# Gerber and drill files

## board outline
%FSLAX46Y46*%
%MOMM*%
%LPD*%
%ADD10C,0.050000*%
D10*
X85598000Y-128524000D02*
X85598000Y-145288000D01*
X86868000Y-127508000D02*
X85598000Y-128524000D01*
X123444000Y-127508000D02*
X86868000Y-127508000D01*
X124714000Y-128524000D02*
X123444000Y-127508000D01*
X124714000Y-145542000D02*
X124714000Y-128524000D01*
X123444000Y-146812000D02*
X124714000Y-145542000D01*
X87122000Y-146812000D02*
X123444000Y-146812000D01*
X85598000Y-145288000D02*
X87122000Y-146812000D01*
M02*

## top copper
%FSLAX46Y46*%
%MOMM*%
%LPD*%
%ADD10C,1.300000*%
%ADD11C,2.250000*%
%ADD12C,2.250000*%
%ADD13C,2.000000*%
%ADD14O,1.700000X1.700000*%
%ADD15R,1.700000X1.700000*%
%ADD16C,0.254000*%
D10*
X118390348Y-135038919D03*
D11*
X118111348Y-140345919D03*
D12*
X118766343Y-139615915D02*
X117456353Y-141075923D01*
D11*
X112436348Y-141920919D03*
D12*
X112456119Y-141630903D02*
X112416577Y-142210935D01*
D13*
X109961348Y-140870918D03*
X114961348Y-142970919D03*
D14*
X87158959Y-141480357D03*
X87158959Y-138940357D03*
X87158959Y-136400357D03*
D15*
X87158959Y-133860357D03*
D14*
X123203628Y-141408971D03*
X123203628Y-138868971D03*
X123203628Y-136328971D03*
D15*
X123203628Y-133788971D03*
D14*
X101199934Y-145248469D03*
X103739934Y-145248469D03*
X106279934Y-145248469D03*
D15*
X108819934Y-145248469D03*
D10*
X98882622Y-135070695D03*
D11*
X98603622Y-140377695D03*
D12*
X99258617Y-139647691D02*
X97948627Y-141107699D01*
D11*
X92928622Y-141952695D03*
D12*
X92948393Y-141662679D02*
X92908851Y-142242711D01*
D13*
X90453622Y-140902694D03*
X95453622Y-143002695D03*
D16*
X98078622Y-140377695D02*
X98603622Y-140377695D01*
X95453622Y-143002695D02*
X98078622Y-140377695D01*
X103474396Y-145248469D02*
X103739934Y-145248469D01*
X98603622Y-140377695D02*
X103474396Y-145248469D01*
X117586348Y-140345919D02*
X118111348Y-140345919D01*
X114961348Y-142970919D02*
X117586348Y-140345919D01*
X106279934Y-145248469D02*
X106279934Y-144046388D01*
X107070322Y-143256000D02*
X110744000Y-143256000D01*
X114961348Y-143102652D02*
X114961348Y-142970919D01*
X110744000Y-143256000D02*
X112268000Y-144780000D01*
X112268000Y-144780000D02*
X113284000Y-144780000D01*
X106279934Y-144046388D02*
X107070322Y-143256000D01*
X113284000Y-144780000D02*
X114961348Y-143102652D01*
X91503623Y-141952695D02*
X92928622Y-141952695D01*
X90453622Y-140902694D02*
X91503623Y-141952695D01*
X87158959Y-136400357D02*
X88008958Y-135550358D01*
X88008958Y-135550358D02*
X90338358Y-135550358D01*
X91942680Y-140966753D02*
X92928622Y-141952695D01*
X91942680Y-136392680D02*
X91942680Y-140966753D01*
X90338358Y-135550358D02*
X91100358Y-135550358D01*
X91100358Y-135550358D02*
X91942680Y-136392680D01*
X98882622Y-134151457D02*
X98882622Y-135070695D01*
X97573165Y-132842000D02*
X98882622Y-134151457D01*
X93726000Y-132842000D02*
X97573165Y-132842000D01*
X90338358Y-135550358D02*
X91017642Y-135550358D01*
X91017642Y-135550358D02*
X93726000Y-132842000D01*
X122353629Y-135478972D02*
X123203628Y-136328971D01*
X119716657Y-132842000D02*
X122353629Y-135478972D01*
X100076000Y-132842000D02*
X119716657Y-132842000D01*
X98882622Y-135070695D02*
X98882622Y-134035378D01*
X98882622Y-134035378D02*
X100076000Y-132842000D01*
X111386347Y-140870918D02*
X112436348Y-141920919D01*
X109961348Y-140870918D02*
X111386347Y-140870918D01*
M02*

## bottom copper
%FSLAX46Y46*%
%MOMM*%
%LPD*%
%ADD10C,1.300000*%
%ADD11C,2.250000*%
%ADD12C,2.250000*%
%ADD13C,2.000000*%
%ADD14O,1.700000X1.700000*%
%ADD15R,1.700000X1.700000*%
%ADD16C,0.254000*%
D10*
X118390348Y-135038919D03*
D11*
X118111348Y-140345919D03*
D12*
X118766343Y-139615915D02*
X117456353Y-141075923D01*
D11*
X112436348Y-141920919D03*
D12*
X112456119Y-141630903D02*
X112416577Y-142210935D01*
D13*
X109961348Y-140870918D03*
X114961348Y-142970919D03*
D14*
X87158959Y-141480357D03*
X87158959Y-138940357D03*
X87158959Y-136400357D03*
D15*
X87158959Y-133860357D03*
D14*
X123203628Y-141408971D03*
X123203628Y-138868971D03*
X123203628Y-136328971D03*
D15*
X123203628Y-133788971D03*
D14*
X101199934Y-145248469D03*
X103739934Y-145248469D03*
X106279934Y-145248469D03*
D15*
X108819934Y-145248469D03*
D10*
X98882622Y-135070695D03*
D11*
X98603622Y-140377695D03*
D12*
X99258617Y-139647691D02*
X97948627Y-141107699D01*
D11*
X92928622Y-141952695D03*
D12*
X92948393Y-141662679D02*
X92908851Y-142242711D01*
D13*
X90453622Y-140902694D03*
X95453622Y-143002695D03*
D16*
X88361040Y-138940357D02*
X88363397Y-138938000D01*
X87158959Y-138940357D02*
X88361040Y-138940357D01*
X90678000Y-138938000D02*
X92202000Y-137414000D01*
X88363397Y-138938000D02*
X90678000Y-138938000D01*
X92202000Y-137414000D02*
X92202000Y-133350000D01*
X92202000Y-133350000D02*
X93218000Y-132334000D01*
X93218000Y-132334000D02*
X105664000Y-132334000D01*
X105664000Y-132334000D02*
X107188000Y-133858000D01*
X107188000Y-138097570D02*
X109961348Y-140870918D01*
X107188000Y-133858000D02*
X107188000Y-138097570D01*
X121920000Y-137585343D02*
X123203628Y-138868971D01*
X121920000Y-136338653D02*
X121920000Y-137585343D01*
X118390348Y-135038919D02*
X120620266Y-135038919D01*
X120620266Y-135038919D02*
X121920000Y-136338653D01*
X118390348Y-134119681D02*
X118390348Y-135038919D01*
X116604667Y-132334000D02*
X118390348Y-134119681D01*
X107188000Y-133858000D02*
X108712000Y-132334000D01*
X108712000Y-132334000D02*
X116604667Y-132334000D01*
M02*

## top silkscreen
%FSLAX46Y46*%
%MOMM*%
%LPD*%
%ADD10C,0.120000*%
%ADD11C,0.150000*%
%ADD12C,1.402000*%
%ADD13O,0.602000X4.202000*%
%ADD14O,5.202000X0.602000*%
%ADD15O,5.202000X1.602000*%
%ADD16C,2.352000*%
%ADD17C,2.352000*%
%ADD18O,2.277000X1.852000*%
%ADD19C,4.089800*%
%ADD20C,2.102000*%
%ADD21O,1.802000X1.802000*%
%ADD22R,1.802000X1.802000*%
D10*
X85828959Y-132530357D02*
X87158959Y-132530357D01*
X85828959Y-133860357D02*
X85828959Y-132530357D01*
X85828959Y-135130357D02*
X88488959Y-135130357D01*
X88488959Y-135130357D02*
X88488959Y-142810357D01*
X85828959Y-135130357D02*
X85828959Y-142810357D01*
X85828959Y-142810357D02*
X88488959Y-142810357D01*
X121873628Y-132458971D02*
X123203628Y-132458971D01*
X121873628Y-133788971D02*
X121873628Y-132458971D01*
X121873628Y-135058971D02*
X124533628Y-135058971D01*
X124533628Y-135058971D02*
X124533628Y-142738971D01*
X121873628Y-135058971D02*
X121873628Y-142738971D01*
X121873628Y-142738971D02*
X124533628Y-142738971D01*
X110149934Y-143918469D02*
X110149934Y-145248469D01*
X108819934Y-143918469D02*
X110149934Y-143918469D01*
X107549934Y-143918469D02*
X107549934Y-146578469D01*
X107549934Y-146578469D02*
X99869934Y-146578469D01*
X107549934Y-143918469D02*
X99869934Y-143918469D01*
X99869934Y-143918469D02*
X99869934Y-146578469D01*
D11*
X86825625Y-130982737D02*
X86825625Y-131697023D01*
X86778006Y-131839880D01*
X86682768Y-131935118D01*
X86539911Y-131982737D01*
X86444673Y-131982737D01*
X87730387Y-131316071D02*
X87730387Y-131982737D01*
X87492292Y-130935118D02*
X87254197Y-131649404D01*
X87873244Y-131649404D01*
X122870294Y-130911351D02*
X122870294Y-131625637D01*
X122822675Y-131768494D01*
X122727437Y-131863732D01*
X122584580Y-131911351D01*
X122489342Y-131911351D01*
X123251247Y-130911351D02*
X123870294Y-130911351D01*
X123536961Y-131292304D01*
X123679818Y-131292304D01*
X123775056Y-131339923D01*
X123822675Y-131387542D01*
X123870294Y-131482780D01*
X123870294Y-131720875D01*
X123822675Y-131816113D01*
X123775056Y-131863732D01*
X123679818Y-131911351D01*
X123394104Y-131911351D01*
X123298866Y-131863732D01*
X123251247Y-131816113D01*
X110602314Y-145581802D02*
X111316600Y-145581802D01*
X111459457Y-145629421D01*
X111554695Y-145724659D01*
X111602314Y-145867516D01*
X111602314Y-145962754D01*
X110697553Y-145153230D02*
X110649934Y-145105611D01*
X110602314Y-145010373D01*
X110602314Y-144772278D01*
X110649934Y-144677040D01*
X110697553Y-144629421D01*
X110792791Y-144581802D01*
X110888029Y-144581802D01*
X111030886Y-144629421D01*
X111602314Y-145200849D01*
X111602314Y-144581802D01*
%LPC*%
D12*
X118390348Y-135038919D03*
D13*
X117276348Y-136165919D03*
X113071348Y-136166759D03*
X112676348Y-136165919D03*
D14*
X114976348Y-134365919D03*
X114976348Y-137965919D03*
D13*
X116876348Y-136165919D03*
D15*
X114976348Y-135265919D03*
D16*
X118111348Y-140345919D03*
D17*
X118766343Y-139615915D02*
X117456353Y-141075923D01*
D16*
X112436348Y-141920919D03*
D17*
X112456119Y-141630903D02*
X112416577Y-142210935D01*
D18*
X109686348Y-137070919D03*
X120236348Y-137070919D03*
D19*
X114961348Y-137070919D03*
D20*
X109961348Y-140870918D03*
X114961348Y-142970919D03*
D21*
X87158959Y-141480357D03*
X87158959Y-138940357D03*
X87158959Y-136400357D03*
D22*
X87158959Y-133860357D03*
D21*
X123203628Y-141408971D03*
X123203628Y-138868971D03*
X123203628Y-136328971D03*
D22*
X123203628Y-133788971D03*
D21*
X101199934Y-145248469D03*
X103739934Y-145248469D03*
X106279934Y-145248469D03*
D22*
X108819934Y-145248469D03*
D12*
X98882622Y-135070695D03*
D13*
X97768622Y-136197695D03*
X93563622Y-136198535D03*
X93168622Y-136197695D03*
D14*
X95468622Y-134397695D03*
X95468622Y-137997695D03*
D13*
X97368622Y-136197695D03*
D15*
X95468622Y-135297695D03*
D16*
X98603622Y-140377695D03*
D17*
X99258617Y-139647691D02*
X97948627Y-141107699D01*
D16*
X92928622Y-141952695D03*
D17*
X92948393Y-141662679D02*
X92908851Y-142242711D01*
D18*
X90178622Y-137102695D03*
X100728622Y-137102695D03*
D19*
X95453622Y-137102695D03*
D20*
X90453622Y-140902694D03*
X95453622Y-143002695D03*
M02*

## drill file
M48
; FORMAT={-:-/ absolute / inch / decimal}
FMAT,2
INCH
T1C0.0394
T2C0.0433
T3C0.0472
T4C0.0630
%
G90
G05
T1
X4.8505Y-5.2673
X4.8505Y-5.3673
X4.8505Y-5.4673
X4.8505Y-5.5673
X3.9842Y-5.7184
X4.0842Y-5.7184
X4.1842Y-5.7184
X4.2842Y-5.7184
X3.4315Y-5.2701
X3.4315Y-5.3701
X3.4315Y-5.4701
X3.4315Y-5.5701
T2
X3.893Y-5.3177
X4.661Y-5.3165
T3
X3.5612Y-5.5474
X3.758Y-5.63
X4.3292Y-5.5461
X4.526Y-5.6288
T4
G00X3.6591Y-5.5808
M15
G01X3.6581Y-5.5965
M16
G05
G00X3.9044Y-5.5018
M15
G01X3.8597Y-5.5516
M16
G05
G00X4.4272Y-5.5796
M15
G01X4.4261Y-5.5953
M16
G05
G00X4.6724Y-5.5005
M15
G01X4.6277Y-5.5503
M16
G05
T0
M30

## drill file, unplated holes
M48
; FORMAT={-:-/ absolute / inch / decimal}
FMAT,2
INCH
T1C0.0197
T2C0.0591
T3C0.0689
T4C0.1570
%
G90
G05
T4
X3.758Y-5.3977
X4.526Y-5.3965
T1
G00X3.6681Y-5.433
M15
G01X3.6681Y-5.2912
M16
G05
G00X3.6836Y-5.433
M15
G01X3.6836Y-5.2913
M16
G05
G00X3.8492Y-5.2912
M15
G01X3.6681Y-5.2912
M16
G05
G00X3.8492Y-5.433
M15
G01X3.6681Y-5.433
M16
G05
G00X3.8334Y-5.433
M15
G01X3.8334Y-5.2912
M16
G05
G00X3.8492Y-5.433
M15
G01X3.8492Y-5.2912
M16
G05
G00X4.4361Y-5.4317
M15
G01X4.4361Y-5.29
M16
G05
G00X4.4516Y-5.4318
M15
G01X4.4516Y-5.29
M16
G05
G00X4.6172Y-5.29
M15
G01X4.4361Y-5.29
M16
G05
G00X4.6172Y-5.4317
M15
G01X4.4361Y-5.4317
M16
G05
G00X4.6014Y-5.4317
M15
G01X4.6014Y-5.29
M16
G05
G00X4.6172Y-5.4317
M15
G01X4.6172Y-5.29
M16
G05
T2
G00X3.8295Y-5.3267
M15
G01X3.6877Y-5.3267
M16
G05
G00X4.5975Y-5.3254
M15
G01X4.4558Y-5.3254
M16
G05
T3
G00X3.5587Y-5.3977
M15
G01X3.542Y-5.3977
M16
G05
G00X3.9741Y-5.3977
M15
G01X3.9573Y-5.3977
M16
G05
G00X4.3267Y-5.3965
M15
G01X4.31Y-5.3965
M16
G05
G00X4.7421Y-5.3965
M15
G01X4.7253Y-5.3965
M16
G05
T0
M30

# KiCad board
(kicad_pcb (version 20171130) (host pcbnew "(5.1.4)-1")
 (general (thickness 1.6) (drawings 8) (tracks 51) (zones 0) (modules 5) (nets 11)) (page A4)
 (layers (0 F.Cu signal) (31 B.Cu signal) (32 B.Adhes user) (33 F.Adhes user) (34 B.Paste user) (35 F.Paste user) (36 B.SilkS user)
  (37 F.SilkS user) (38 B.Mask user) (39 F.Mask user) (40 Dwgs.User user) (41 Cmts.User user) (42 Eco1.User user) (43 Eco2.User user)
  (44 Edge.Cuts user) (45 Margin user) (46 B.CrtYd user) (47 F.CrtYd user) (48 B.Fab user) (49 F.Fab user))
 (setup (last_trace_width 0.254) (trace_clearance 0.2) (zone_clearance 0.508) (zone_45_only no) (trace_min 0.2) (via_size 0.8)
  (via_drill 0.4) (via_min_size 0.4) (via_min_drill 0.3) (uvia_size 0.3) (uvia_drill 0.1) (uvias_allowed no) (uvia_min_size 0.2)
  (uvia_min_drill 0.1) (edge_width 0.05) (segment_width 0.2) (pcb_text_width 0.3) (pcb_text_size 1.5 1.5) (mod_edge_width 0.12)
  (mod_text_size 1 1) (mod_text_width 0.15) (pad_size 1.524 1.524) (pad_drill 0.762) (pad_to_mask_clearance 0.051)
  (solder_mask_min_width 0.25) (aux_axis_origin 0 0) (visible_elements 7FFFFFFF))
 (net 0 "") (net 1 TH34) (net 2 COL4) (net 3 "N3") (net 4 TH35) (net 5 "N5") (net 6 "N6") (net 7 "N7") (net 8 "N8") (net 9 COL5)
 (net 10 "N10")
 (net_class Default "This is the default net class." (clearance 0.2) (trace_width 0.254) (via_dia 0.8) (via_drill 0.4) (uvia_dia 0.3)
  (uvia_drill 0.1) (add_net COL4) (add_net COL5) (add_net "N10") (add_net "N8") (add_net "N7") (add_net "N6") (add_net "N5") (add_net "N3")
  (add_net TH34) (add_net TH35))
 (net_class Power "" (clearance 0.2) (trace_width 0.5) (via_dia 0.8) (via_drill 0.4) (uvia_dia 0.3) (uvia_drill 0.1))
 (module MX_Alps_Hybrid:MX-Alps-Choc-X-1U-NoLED (layer F.Cu) (at 114.961348 137.070919 180)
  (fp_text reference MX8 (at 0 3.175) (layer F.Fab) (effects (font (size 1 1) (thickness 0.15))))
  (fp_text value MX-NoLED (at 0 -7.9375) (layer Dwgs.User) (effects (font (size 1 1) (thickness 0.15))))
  (pad 1 thru_hole circle (at -3.429 2.032 180) (size 1.3 1.3) (drill 1.1) (layers *.Cu *.Mask) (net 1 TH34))
  (pad "" np_thru_hole oval (at -2.315 0.905 180) (size 0.5 4.1) (drill oval 0.5 4.1) (layers *.Cu *.Mask))
  (pad "" np_thru_hole oval (at 1.89 0.90416 180) (size 0.5 4.1) (drill oval 0.5 4.1) (layers *.Cu *.Mask))
  (pad "" np_thru_hole oval (at 2.285 0.905 180) (size 0.5 4.1) (drill oval 0.5 4.1) (layers *.Cu *.Mask))
  (pad "" np_thru_hole oval (at -0.015 2.705 180) (size 5.1 0.5) (drill oval 5.1 0.5) (layers *.Cu *.Mask))
  (pad "" np_thru_hole oval (at -0.015 -0.895 180) (size 5.1 0.5) (drill oval 5.1 0.5) (layers *.Cu *.Mask))
  (pad "" np_thru_hole oval (at -1.915 0.905 180) (size 0.5 4.1) (drill oval 0.5 4.1) (layers *.Cu *.Mask))
  (pad "" np_thru_hole oval (at -0.015 1.805 180) (size 5.1 1.5) (drill oval 5.1 1.5) (layers *.Cu *.Mask))
  (pad 2 thru_hole oval (at -3.15 -3.275 228.1) (size 4.211556 2.25) (drill oval 3.3 1.6) (layers *.Cu *.Mask) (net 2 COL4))
  (pad 1 thru_hole oval (at 2.525 -4.85 266.1) (size 2.831378 2.25) (drill oval 2 1.6) (layers *.Cu *.Mask) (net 1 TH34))
  (pad "" np_thru_hole oval (at 5.275 0 270) (size 1.75 2.175) (drill oval 1.75 2.175) (layers *.Cu *.Mask))
  (pad "" np_thru_hole oval (at -5.275 0 270) (size 1.75 2.175) (drill oval 1.75 2.175) (layers *.Cu *.Mask))
  (pad "" np_thru_hole circle (at 0 0 180) (size 3.9878 3.9878) (drill 3.9878) (layers *.Cu *.Mask))
  (pad 1 thru_hole circle (at 5 -3.799999 180) (size 2 2) (drill 1.2) (layers *.Cu *.Mask) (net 1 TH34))
  (pad 2 thru_hole circle (at 0 -5.9 180) (size 2 2) (drill 1.2) (layers *.Cu *.Mask) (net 2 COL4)))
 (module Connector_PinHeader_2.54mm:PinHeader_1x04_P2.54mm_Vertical (layer F.Cu) (at 87.158959 133.860357)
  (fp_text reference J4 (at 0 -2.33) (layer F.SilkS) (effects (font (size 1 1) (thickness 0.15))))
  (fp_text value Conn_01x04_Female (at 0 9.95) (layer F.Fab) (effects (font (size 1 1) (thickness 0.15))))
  (fp_line (start -1.33 -1.33) (end 0 -1.33) (layer F.SilkS) (width 0.12))
  (fp_line (start -1.33 0) (end -1.33 -1.33) (layer F.SilkS) (width 0.12))
  (fp_line (start -1.33 1.27) (end 1.33 1.27) (layer F.SilkS) (width 0.12))
  (fp_line (start 1.33 1.27) (end 1.33 8.95) (layer F.SilkS) (width 0.12))
  (fp_line (start -1.33 1.27) (end -1.33 8.95) (layer F.SilkS) (width 0.12))
  (fp_line (start -1.33 8.95) (end 1.33 8.95) (layer F.SilkS) (width 0.12))
  (pad 4 thru_hole oval (at 0 7.62) (size 1.7 1.7) (drill 1) (layers *.Cu *.Mask) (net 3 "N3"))
  (pad 3 thru_hole oval (at 0 5.08) (size 1.7 1.7) (drill 1) (layers *.Cu *.Mask) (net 1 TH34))
  (pad 2 thru_hole oval (at 0 2.54) (size 1.7 1.7) (drill 1) (layers *.Cu *.Mask) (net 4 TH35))
  (pad 1 thru_hole rect (at 0 0) (size 1.7 1.7) (drill 1) (layers *.Cu *.Mask) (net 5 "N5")))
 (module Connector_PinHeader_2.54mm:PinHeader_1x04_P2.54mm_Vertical (layer F.Cu) (at 123.203628 133.788971)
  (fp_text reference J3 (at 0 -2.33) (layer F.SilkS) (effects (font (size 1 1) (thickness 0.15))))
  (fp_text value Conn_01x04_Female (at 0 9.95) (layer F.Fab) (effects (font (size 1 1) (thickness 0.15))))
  (fp_line (start -1.33 -1.33) (end 0 -1.33) (layer F.SilkS) (width 0.12))
  (fp_line (start -1.33 0) (end -1.33 -1.33) (layer F.SilkS) (width 0.12))
  (fp_line (start -1.33 1.27) (end 1.33 1.27) (layer F.SilkS) (width 0.12))
  (fp_line (start 1.33 1.27) (end 1.33 8.95) (layer F.SilkS) (width 0.12))
  (fp_line (start -1.33 1.27) (end -1.33 8.95) (layer F.SilkS) (width 0.12))
  (fp_line (start -1.33 8.95) (end 1.33 8.95) (layer F.SilkS) (width 0.12))
  (pad 4 thru_hole oval (at 0 7.62) (size 1.7 1.7) (drill 1) (layers *.Cu *.Mask) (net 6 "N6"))
  (pad 3 thru_hole oval (at 0 5.08) (size 1.7 1.7) (drill 1) (layers *.Cu *.Mask) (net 1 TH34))
  (pad 2 thru_hole oval (at 0 2.54) (size 1.7 1.7) (drill 1) (layers *.Cu *.Mask) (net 4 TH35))
  (pad 1 thru_hole rect (at 0 0) (size 1.7 1.7) (drill 1) (layers *.Cu *.Mask) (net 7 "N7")))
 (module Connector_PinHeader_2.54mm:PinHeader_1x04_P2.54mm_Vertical (layer F.Cu) (at 108.819934 145.248469 270)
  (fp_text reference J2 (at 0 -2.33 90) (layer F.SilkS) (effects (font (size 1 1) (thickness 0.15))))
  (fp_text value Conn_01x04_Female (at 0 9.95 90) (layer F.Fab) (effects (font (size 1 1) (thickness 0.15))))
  (fp_line (start -1.33 -1.33) (end 0 -1.33) (layer F.SilkS) (width 0.12))
  (fp_line (start -1.33 0) (end -1.33 -1.33) (layer F.SilkS) (width 0.12))
  (fp_line (start -1.33 1.27) (end 1.33 1.27) (layer F.SilkS) (width 0.12))
  (fp_line (start 1.33 1.27) (end 1.33 8.95) (layer F.SilkS) (width 0.12))
  (fp_line (start -1.33 1.27) (end -1.33 8.95) (layer F.SilkS) (width 0.12))
  (fp_line (start -1.33 8.95) (end 1.33 8.95) (layer F.SilkS) (width 0.12))
  (pad 4 thru_hole oval (at 0 7.62 270) (size 1.7 1.7) (drill 1) (layers *.Cu *.Mask) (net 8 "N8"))
  (pad 3 thru_hole oval (at 0 5.08 270) (size 1.7 1.7) (drill 1) (layers *.Cu *.Mask) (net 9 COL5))
  (pad 2 thru_hole oval (at 0 2.54 270) (size 1.7 1.7) (drill 1) (layers *.Cu *.Mask) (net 2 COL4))
  (pad 1 thru_hole rect (at 0 0 270) (size 1.7 1.7) (drill 1) (layers *.Cu *.Mask) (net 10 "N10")))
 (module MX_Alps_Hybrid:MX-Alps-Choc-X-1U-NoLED (layer F.Cu) (at 95.453622 137.102695 180)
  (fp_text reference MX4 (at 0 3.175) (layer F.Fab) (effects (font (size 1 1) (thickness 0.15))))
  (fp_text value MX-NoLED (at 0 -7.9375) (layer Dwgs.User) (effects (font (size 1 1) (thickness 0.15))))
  (pad 1 thru_hole circle (at -3.429 2.032 180) (size 1.3 1.3) (drill 1.1) (layers *.Cu *.Mask) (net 4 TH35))
  (pad "" np_thru_hole oval (at -2.315 0.905 180) (size 0.5 4.1) (drill oval 0.5 4.1) (layers *.Cu *.Mask))
  (pad "" np_thru_hole oval (at 1.89 0.90416 180) (size 0.5 4.1) (drill oval 0.5 4.1) (layers *.Cu *.Mask))
  (pad "" np_thru_hole oval (at 2.285 0.905 180) (size 0.5 4.1) (drill oval 0.5 4.1) (layers *.Cu *.Mask))
  (pad "" np_thru_hole oval (at -0.015 2.705 180) (size 5.1 0.5) (drill oval 5.1 0.5) (layers *.Cu *.Mask))
  (pad "" np_thru_hole oval (at -0.015 -0.895 180) (size 5.1 0.5) (drill oval 5.1 0.5) (layers *.Cu *.Mask))
  (pad "" np_thru_hole oval (at -1.915 0.905 180) (size 0.5 4.1) (drill oval 0.5 4.1) (layers *.Cu *.Mask))
  (pad "" np_thru_hole oval (at -0.015 1.805 180) (size 5.1 1.5) (drill oval 5.1 1.5) (layers *.Cu *.Mask))
  (pad 2 thru_hole oval (at -3.15 -3.275 228.1) (size 4.211556 2.25) (drill oval 3.3 1.6) (layers *.Cu *.Mask) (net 9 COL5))
  (pad 1 thru_hole oval (at 2.525 -4.85 266.1) (size 2.831378 2.25) (drill oval 2 1.6) (layers *.Cu *.Mask) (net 4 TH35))
  (pad "" np_thru_hole oval (at 5.275 0 270) (size 1.75 2.175) (drill oval 1.75 2.175) (layers *.Cu *.Mask))
  (pad "" np_thru_hole oval (at -5.275 0 270) (size 1.75 2.175) (drill oval 1.75 2.175) (layers *.Cu *.Mask))
  (pad "" np_thru_hole circle (at 0 0 180) (size 3.9878 3.9878) (drill 3.9878) (layers *.Cu *.Mask))
  (pad 1 thru_hole circle (at 5 -3.799999 180) (size 2 2) (drill 1.2) (layers *.Cu *.Mask) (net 4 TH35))
  (pad 2 thru_hole circle (at 0 -5.9 180) (size 2 2) (drill 1.2) (layers *.Cu *.Mask) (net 9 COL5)))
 (gr_line (start 85.598 128.524) (end 85.598 145.288) (layer Edge.Cuts) (width 0.05))
 (gr_line (start 86.868 127.508) (end 85.598 128.524) (layer Edge.Cuts) (width 0.05))
 (gr_line (start 123.444 127.508) (end 86.868 127.508) (layer Edge.Cuts) (width 0.05))
 (gr_line (start 124.714 128.524) (end 123.444 127.508) (layer Edge.Cuts) (width 0.05))
 (gr_line (start 124.714 145.542) (end 124.714 128.524) (layer Edge.Cuts) (width 0.05))
 (gr_line (start 123.444 146.812) (end 124.714 145.542) (layer Edge.Cuts) (width 0.05))
 (gr_line (start 87.122 146.812) (end 123.444 146.812) (layer Edge.Cuts) (width 0.05))
 (gr_line (start 85.598 145.288) (end 87.122 146.812) (layer Edge.Cuts) (width 0.05))
 (segment (start 98.078622 140.377695) (end 98.603622 140.377695) (width 0.254) (layer F.Cu) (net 9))
 (segment (start 95.453622 143.002695) (end 98.078622 140.377695) (width 0.254) (layer F.Cu) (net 9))
 (segment (start 103.474396 145.248469) (end 103.739934 145.248469) (width 0.254) (layer F.Cu) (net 9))
 (segment (start 98.603622 140.377695) (end 103.474396 145.248469) (width 0.254) (layer F.Cu) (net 9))
 (segment (start 117.586348 140.345919) (end 118.111348 140.345919) (width 0.254) (layer F.Cu) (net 2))
 (segment (start 114.961348 142.970919) (end 117.586348 140.345919) (width 0.254) (layer F.Cu) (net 2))
 (segment (start 106.279934 145.248469) (end 106.279934 144.046388) (width 0.254) (layer F.Cu) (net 2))
 (segment (start 107.070322 143.256) (end 110.744 143.256) (width 0.254) (layer F.Cu) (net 2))
 (segment (start 114.961348 143.102652) (end 114.961348 142.970919) (width 0.254) (layer F.Cu) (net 2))
 (segment (start 110.744 143.256) (end 112.268 144.78) (width 0.254) (layer F.Cu) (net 2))
 (segment (start 112.268 144.78) (end 113.284 144.78) (width 0.254) (layer F.Cu) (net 2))
 (segment (start 106.279934 144.046388) (end 107.070322 143.256) (width 0.254) (layer F.Cu) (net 2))
 (segment (start 113.284 144.78) (end 114.961348 143.102652) (width 0.254) (layer F.Cu) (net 2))
 (segment (start 91.503623 141.952695) (end 92.928622 141.952695) (width 0.254) (layer F.Cu) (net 4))
 (segment (start 90.453622 140.902694) (end 91.503623 141.952695) (width 0.254) (layer F.Cu) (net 4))
 (segment (start 87.158959 136.400357) (end 88.008958 135.550358) (width 0.254) (layer F.Cu) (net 4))
 (segment (start 88.008958 135.550358) (end 90.338358 135.550358) (width 0.254) (layer F.Cu) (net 4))
 (segment (start 91.94268 140.966753) (end 92.928622 141.952695) (width 0.254) (layer F.Cu) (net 4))
 (segment (start 91.94268 136.39268) (end 91.94268 140.966753) (width 0.254) (layer F.Cu) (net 4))
 (segment (start 90.338358 135.550358) (end 91.100358 135.550358) (width 0.254) (layer F.Cu) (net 4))
 (segment (start 91.100358 135.550358) (end 91.94268 136.39268) (width 0.254) (layer F.Cu) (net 4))
 (segment (start 98.882622 134.151457) (end 98.882622 135.070695) (width 0.254) (layer F.Cu) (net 4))
 (segment (start 97.573165 132.842) (end 98.882622 134.151457) (width 0.254) (layer F.Cu) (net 4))
 (segment (start 93.726 132.842) (end 97.573165 132.842) (width 0.254) (layer F.Cu) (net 4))
 (segment (start 90.338358 135.550358) (end 91.017642 135.550358) (width 0.254) (layer F.Cu) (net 4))
 (segment (start 91.017642 135.550358) (end 93.726 132.842) (width 0.254) (layer F.Cu) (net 4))
 (segment (start 122.353629 135.478972) (end 123.203628 136.328971) (width 0.254) (layer F.Cu) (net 4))
 (segment (start 119.716657 132.842) (end 122.353629 135.478972) (width 0.254) (layer F.Cu) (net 4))
 (segment (start 100.076 132.842) (end 119.716657 132.842) (width 0.254) (layer F.Cu) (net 4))
 (segment (start 98.882622 135.070695) (end 98.882622 134.035378) (width 0.254) (layer F.Cu) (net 4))
 (segment (start 98.882622 134.035378) (end 100.076 132.842) (width 0.254) (layer F.Cu) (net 4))
 (segment (start 111.386347 140.870918) (end 112.436348 141.920919) (width 0.254) (layer F.Cu) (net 1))
 (segment (start 109.961348 140.870918) (end 111.386347 140.870918) (width 0.254) (layer F.Cu) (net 1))
 (segment (start 88.36104 138.940357) (end 88.363397 138.938) (width 0.254) (layer B.Cu) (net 1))
 (segment (start 87.158959 138.940357) (end 88.36104 138.940357) (width 0.254) (layer B.Cu) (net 1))
 (segment (start 90.678 138.938) (end 92.202 137.414) (width 0.254) (layer B.Cu) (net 1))
 (segment (start 88.363397 138.938) (end 90.678 138.938) (width 0.254) (layer B.Cu) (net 1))
 (segment (start 92.202 137.414) (end 92.202 133.35) (width 0.254) (layer B.Cu) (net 1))
 (segment (start 92.202 133.35) (end 93.218 132.334) (width 0.254) (layer B.Cu) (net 1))
 (segment (start 93.218 132.334) (end 105.664 132.334) (width 0.254) (layer B.Cu) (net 1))
 (segment (start 105.664 132.334) (end 107.188 133.858) (width 0.254) (layer B.Cu) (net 1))
 (segment (start 107.188 138.09757) (end 109.961348 140.870918) (width 0.254) (layer B.Cu) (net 1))
 (segment (start 107.188 133.858) (end 107.188 138.09757) (width 0.254) (layer B.Cu) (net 1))
 (segment (start 121.92 137.585343) (end 123.203628 138.868971) (width 0.254) (layer B.Cu) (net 1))
 (segment (start 121.92 136.338653) (end 121.92 137.585343) (width 0.254) (layer B.Cu) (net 1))
 (segment (start 118.390348 135.038919) (end 120.620266 135.038919) (width 0.254) (layer B.Cu) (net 1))
 (segment (start 120.620266 135.038919) (end 121.92 136.338653) (width 0.254) (layer B.Cu) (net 1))
 (segment (start 118.390348 134.119681) (end 118.390348 135.038919) (width 0.254) (layer B.Cu) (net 1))
 (segment (start 116.604667 132.334) (end 118.390348 134.119681) (width 0.254) (layer B.Cu) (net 1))
 (segment (start 107.188 133.858) (end 108.712 132.334) (width 0.254) (layer B.Cu) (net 1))
 (segment (start 108.712 132.334) (end 116.604667 132.334) (width 0.254) (layer B.Cu) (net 1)))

